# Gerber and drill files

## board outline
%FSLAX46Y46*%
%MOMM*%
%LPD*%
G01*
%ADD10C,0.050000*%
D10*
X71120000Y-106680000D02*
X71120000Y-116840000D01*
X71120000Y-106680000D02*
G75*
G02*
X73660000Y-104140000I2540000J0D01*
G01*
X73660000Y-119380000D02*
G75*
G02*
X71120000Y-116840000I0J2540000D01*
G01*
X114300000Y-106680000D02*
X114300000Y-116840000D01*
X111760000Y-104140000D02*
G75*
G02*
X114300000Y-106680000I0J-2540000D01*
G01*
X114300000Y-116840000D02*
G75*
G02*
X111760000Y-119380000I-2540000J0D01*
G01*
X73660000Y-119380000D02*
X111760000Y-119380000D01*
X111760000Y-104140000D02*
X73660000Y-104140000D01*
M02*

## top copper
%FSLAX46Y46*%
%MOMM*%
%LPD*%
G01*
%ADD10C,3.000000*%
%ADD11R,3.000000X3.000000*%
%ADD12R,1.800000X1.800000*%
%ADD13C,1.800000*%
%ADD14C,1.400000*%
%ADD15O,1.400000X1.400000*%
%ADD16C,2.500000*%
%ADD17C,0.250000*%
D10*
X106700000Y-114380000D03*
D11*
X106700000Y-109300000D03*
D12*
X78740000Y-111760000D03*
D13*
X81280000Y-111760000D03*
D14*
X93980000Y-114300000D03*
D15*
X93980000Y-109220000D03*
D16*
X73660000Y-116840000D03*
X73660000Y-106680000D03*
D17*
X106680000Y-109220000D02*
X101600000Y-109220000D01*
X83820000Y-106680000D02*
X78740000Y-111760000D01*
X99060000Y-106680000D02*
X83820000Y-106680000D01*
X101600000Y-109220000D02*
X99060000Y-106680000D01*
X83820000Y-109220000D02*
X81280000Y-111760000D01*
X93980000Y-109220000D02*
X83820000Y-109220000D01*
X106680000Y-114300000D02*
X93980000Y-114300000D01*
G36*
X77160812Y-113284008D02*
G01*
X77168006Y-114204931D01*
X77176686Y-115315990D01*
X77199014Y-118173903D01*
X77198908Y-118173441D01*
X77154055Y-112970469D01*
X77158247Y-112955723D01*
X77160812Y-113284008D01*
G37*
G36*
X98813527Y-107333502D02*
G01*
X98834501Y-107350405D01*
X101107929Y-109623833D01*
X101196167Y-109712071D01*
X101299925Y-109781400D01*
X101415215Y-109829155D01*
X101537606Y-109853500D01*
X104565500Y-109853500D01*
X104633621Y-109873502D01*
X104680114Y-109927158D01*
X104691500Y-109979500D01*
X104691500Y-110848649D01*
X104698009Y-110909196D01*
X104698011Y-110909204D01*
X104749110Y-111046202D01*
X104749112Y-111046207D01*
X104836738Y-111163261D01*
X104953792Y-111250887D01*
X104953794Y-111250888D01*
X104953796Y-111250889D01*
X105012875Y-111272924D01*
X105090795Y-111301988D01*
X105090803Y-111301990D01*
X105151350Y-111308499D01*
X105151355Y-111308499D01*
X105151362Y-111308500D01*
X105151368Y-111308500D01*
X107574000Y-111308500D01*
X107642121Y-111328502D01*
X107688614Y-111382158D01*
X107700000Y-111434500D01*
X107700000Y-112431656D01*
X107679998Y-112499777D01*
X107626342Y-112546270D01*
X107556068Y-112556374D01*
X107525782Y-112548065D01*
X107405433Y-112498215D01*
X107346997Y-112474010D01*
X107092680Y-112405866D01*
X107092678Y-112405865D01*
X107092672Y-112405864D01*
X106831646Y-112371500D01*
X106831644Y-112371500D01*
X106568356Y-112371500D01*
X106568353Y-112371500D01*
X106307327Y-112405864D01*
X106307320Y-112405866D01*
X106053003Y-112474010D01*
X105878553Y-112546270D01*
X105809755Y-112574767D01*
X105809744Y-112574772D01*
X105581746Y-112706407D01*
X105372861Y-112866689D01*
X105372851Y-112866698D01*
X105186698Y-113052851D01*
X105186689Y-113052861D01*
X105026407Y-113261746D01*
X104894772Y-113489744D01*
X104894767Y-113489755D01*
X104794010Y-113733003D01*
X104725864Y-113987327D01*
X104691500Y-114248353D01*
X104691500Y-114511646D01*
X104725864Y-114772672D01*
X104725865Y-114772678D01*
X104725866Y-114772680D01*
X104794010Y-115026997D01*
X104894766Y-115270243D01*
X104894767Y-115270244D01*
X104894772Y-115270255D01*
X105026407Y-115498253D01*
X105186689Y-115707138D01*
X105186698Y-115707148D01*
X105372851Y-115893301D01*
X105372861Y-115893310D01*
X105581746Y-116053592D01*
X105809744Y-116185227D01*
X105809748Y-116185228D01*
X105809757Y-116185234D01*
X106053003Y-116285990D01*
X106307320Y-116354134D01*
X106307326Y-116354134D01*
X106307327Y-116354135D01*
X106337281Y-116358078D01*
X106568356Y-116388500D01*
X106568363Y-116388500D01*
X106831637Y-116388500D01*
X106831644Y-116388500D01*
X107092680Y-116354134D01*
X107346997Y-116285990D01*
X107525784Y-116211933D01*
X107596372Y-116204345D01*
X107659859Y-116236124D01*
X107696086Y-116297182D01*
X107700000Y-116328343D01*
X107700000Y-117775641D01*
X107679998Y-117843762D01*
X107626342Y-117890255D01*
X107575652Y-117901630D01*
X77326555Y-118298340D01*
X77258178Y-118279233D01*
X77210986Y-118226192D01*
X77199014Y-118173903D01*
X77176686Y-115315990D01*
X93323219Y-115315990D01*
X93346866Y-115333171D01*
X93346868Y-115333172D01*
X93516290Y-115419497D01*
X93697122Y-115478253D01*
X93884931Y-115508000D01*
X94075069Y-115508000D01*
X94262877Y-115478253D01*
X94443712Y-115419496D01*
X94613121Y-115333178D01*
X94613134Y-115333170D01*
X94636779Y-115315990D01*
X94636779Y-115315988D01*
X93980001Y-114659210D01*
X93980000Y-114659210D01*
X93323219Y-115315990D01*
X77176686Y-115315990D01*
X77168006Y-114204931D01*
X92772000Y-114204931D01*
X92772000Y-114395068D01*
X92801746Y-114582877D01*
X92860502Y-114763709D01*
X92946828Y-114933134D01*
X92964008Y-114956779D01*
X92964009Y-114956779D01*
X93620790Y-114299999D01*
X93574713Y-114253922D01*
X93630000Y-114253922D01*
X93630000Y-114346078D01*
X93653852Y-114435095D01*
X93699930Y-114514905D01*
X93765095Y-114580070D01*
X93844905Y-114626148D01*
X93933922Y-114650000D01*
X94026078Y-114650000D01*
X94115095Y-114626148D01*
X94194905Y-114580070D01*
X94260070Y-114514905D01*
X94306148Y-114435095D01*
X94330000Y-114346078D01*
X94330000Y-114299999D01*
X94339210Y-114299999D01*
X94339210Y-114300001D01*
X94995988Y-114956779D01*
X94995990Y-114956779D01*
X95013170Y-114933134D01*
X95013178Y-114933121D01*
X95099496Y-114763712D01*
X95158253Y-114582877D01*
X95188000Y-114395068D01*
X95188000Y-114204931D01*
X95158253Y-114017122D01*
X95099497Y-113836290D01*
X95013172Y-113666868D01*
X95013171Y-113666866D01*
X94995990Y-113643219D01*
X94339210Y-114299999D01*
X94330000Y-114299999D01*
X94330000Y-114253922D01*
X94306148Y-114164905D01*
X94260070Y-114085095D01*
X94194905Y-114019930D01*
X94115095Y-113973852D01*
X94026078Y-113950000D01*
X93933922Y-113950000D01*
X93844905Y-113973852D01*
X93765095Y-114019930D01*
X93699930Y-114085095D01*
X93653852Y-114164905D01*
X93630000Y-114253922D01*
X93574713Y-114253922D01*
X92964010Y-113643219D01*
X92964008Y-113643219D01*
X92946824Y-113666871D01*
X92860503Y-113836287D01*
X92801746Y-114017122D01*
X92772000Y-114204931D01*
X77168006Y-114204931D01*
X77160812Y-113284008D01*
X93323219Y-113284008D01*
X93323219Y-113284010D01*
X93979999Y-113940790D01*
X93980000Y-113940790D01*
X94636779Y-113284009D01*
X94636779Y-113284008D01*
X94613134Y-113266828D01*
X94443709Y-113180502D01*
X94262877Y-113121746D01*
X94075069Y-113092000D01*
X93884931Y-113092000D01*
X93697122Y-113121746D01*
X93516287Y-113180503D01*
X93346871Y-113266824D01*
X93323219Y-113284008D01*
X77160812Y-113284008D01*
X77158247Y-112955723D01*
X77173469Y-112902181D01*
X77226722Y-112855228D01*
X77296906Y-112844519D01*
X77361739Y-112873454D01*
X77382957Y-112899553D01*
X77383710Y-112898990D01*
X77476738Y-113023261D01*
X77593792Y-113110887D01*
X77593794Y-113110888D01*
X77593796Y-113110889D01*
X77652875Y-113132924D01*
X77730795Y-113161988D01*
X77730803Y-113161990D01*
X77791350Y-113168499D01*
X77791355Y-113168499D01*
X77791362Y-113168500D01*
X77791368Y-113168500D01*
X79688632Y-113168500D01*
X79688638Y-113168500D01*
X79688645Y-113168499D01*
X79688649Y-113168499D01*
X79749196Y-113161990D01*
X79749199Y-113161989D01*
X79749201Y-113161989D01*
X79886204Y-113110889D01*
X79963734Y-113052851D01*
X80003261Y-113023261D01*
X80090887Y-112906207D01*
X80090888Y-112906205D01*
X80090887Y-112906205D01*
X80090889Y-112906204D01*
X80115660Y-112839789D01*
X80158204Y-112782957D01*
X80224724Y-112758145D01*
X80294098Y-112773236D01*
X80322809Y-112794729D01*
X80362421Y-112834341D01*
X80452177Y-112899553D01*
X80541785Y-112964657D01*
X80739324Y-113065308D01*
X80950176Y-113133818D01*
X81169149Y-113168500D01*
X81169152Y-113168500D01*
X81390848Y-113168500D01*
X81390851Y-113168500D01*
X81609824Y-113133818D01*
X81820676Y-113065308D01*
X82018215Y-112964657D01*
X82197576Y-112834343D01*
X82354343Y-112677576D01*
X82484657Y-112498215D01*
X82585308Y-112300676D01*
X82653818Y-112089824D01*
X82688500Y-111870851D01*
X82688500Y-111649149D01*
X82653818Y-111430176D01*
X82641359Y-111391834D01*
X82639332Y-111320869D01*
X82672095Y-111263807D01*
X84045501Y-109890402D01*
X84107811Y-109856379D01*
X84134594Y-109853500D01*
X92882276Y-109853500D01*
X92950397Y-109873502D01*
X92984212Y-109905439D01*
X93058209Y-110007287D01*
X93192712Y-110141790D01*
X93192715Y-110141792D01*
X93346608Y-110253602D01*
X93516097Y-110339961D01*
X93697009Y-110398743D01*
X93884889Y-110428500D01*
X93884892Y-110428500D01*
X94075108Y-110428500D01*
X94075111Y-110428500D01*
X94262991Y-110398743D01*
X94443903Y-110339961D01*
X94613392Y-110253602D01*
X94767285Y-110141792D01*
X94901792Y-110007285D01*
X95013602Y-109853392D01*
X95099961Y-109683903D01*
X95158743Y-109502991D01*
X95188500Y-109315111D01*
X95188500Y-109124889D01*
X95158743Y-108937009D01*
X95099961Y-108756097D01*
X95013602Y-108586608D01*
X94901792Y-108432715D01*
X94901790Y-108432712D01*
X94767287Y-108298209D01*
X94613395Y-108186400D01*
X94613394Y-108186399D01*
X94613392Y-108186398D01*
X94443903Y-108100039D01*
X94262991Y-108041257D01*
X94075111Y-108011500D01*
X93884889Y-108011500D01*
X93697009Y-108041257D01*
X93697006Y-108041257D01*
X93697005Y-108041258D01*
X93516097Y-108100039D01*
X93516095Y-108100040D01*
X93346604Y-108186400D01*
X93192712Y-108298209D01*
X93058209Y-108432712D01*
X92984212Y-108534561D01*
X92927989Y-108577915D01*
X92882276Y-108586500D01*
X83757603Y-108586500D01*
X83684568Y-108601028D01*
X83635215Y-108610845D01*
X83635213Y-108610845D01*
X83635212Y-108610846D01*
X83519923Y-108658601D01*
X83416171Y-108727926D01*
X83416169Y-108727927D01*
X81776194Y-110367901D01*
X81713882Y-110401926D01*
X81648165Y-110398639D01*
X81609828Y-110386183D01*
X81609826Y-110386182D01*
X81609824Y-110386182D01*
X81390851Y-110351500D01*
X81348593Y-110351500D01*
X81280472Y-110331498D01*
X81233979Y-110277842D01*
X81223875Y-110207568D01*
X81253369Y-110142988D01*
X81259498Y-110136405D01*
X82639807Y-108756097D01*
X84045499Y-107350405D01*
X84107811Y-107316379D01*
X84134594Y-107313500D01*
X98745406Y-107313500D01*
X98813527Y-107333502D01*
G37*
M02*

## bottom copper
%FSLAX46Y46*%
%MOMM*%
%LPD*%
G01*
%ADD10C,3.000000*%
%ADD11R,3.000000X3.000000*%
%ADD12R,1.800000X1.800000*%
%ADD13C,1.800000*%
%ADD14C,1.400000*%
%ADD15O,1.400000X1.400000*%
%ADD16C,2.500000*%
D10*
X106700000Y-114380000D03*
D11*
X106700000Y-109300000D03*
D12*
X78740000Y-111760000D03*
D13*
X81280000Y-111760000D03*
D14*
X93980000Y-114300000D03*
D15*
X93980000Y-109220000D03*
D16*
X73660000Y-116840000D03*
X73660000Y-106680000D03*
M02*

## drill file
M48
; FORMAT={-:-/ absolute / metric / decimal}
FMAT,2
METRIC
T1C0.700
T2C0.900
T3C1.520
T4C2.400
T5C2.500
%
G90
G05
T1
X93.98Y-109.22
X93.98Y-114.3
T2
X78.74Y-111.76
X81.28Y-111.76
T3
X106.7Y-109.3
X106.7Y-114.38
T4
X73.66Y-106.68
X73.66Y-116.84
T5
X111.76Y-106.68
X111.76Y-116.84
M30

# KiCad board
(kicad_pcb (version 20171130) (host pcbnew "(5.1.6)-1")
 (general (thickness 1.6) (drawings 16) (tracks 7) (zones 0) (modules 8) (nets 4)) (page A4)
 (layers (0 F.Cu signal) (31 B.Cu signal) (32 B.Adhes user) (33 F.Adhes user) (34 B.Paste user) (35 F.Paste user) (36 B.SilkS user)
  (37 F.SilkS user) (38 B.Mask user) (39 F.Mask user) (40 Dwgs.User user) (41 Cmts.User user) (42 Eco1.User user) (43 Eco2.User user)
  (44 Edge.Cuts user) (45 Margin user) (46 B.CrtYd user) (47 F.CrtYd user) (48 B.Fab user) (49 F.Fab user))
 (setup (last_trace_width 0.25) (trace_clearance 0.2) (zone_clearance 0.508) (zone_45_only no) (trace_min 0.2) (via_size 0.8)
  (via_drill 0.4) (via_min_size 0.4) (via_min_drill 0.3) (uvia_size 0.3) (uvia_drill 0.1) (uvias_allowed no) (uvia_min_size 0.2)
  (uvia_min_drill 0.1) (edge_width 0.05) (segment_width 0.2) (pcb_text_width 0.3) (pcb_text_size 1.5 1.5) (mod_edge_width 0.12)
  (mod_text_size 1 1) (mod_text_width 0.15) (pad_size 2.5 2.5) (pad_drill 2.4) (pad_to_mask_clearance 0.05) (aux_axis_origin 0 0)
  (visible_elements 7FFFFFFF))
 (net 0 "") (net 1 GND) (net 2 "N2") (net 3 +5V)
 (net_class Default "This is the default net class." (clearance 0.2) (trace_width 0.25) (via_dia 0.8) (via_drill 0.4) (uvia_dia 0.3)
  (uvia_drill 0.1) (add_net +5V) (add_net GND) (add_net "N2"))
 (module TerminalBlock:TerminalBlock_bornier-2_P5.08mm (layer F.Cu) (at 106.7 109.3 270)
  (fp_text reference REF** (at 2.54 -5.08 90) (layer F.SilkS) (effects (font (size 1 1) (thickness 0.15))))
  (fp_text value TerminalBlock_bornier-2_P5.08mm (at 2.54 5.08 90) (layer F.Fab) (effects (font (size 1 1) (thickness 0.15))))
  (pad 2 thru_hole circle (at 5.08 0 270) (size 3 3) (drill 1.52) (layers *.Cu *.Mask))
  (pad 2 thru_hole rect (at 0 0 270) (size 3 3) (drill 1.52) (layers *.Cu *.Mask)))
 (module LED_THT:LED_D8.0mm (layer F.Cu) (at 78.74 111.76)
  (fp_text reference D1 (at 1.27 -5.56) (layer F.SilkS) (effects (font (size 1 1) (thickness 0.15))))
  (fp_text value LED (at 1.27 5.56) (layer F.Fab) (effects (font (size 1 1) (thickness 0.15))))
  (pad 1 thru_hole rect (at 0 0) (size 1.8 1.8) (drill 0.9) (layers *.Cu *.Mask) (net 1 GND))
  (pad 2 thru_hole circle (at 2.54 0) (size 1.8 1.8) (drill 0.9) (layers *.Cu *.Mask) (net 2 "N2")))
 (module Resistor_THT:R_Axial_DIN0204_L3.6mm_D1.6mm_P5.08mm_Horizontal (layer F.Cu) (at 93.98 114.3 90)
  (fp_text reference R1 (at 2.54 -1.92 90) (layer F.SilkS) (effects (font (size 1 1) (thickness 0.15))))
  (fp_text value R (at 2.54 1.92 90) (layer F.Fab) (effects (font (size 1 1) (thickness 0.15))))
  (pad 1 thru_hole circle (at 0 0 90) (size 1.4 1.4) (drill 0.7) (layers *.Cu *.Mask) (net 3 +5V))
  (pad 2 thru_hole oval (at 5.08 0 90) (size 1.4 1.4) (drill 0.7) (layers *.Cu *.Mask) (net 2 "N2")))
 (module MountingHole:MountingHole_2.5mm (layer F.Cu) (at 73.66 116.84)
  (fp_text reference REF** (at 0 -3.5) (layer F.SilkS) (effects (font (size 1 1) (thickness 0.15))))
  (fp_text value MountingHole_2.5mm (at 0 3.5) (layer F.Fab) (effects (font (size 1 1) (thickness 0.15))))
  (pad "" np_thru_hole circle (at 0 0) (size 2.5 2.5) (drill 2.4) (layers *.Cu *.Mask)))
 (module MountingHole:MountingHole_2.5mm (layer F.Cu) (at 73.66 106.68)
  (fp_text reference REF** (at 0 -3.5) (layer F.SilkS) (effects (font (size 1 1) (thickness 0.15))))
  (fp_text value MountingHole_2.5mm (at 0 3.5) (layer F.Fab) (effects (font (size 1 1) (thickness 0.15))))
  (pad "" np_thru_hole circle (at 0 0) (size 2.5 2.5) (drill 2.4) (layers *.Cu *.Mask)))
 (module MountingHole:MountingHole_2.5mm (layer F.Cu) (at 111.76 106.68)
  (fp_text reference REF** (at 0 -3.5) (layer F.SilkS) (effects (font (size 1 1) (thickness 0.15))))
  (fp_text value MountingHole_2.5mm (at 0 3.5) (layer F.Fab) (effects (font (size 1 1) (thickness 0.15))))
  (pad 1 np_thru_hole circle (at 0 0) (size 2.5 2.5) (drill 2.5) (layers *.Cu *.Mask)))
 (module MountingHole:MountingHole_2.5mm (layer F.Cu) (at 111.76 116.84)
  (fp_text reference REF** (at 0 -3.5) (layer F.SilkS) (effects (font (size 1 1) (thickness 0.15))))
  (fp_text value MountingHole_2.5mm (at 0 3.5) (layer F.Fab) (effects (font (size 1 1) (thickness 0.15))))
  (pad 1 np_thru_hole circle (at 0 0) (size 2.5 2.5) (drill 2.5) (layers *.Cu *.Mask)))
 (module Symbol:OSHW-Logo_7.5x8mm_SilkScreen (layer B.Cu) (at 81.6 113.6 180)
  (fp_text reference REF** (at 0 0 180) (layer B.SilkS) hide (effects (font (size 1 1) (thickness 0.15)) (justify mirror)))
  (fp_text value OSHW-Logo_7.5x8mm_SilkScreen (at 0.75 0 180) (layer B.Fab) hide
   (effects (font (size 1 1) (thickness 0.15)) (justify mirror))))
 (gr_line (start 71.12 106.68) (end 71.12 116.84) (angle 90) (layer Edge.Cuts) (width 0.05))
 (gr_arc (start 73.66 106.68) (end 71.12 106.68) (angle 90) (layer Edge.Cuts) (width 0.05))
 (gr_arc (start 73.66 116.84) (end 73.66 119.38) (angle 90) (layer Edge.Cuts) (width 0.05))
 (gr_line (start 114.3 106.68) (end 114.3 116.84) (angle 90) (layer Edge.Cuts) (width 0.05))
 (gr_arc (start 111.76 106.68) (end 111.76 104.14) (angle 90) (layer Edge.Cuts) (width 0.05))
 (gr_arc (start 111.76 116.84) (end 114.3 116.84) (angle 90) (layer Edge.Cuts) (width 0.05))
 (gr_line (start 73.66 119.38) (end 111.76 119.38) (angle 90) (layer Edge.Cuts) (width 0.05))
 (gr_line (start 111.76 104.14) (end 73.66 104.14) (angle 90) (layer Edge.Cuts) (width 0.05))
 (segment (start 106.68 109.22) (end 101.6 109.22) (width 0.25) (layer F.Cu) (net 1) (status 400000))
 (segment (start 83.82 106.68) (end 78.74 111.76) (width 0.25) (layer F.Cu) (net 1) (status 800000))
 (segment (start 99.06 106.68) (end 83.82 106.68) (width 0.25) (layer F.Cu) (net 1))
 (segment (start 101.6 109.22) (end 99.06 106.68) (width 0.25) (layer F.Cu) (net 1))
 (segment (start 83.82 109.22) (end 81.28 111.76) (width 0.25) (layer F.Cu) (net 2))
 (segment (start 93.98 109.22) (end 83.82 109.22) (width 0.25) (layer F.Cu) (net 2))
 (segment (start 106.68 114.3) (end 93.98 114.3) (width 0.25) (layer F.Cu) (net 3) (status C00000))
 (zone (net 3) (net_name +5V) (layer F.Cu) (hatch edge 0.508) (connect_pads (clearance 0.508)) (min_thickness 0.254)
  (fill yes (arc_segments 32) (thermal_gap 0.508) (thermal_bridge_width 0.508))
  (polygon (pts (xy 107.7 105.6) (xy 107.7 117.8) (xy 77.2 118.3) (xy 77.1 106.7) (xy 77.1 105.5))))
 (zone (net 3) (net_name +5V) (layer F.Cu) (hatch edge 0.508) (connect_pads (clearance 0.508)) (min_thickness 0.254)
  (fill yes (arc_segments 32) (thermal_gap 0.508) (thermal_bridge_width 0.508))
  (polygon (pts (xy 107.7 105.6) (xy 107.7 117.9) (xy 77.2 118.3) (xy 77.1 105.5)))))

